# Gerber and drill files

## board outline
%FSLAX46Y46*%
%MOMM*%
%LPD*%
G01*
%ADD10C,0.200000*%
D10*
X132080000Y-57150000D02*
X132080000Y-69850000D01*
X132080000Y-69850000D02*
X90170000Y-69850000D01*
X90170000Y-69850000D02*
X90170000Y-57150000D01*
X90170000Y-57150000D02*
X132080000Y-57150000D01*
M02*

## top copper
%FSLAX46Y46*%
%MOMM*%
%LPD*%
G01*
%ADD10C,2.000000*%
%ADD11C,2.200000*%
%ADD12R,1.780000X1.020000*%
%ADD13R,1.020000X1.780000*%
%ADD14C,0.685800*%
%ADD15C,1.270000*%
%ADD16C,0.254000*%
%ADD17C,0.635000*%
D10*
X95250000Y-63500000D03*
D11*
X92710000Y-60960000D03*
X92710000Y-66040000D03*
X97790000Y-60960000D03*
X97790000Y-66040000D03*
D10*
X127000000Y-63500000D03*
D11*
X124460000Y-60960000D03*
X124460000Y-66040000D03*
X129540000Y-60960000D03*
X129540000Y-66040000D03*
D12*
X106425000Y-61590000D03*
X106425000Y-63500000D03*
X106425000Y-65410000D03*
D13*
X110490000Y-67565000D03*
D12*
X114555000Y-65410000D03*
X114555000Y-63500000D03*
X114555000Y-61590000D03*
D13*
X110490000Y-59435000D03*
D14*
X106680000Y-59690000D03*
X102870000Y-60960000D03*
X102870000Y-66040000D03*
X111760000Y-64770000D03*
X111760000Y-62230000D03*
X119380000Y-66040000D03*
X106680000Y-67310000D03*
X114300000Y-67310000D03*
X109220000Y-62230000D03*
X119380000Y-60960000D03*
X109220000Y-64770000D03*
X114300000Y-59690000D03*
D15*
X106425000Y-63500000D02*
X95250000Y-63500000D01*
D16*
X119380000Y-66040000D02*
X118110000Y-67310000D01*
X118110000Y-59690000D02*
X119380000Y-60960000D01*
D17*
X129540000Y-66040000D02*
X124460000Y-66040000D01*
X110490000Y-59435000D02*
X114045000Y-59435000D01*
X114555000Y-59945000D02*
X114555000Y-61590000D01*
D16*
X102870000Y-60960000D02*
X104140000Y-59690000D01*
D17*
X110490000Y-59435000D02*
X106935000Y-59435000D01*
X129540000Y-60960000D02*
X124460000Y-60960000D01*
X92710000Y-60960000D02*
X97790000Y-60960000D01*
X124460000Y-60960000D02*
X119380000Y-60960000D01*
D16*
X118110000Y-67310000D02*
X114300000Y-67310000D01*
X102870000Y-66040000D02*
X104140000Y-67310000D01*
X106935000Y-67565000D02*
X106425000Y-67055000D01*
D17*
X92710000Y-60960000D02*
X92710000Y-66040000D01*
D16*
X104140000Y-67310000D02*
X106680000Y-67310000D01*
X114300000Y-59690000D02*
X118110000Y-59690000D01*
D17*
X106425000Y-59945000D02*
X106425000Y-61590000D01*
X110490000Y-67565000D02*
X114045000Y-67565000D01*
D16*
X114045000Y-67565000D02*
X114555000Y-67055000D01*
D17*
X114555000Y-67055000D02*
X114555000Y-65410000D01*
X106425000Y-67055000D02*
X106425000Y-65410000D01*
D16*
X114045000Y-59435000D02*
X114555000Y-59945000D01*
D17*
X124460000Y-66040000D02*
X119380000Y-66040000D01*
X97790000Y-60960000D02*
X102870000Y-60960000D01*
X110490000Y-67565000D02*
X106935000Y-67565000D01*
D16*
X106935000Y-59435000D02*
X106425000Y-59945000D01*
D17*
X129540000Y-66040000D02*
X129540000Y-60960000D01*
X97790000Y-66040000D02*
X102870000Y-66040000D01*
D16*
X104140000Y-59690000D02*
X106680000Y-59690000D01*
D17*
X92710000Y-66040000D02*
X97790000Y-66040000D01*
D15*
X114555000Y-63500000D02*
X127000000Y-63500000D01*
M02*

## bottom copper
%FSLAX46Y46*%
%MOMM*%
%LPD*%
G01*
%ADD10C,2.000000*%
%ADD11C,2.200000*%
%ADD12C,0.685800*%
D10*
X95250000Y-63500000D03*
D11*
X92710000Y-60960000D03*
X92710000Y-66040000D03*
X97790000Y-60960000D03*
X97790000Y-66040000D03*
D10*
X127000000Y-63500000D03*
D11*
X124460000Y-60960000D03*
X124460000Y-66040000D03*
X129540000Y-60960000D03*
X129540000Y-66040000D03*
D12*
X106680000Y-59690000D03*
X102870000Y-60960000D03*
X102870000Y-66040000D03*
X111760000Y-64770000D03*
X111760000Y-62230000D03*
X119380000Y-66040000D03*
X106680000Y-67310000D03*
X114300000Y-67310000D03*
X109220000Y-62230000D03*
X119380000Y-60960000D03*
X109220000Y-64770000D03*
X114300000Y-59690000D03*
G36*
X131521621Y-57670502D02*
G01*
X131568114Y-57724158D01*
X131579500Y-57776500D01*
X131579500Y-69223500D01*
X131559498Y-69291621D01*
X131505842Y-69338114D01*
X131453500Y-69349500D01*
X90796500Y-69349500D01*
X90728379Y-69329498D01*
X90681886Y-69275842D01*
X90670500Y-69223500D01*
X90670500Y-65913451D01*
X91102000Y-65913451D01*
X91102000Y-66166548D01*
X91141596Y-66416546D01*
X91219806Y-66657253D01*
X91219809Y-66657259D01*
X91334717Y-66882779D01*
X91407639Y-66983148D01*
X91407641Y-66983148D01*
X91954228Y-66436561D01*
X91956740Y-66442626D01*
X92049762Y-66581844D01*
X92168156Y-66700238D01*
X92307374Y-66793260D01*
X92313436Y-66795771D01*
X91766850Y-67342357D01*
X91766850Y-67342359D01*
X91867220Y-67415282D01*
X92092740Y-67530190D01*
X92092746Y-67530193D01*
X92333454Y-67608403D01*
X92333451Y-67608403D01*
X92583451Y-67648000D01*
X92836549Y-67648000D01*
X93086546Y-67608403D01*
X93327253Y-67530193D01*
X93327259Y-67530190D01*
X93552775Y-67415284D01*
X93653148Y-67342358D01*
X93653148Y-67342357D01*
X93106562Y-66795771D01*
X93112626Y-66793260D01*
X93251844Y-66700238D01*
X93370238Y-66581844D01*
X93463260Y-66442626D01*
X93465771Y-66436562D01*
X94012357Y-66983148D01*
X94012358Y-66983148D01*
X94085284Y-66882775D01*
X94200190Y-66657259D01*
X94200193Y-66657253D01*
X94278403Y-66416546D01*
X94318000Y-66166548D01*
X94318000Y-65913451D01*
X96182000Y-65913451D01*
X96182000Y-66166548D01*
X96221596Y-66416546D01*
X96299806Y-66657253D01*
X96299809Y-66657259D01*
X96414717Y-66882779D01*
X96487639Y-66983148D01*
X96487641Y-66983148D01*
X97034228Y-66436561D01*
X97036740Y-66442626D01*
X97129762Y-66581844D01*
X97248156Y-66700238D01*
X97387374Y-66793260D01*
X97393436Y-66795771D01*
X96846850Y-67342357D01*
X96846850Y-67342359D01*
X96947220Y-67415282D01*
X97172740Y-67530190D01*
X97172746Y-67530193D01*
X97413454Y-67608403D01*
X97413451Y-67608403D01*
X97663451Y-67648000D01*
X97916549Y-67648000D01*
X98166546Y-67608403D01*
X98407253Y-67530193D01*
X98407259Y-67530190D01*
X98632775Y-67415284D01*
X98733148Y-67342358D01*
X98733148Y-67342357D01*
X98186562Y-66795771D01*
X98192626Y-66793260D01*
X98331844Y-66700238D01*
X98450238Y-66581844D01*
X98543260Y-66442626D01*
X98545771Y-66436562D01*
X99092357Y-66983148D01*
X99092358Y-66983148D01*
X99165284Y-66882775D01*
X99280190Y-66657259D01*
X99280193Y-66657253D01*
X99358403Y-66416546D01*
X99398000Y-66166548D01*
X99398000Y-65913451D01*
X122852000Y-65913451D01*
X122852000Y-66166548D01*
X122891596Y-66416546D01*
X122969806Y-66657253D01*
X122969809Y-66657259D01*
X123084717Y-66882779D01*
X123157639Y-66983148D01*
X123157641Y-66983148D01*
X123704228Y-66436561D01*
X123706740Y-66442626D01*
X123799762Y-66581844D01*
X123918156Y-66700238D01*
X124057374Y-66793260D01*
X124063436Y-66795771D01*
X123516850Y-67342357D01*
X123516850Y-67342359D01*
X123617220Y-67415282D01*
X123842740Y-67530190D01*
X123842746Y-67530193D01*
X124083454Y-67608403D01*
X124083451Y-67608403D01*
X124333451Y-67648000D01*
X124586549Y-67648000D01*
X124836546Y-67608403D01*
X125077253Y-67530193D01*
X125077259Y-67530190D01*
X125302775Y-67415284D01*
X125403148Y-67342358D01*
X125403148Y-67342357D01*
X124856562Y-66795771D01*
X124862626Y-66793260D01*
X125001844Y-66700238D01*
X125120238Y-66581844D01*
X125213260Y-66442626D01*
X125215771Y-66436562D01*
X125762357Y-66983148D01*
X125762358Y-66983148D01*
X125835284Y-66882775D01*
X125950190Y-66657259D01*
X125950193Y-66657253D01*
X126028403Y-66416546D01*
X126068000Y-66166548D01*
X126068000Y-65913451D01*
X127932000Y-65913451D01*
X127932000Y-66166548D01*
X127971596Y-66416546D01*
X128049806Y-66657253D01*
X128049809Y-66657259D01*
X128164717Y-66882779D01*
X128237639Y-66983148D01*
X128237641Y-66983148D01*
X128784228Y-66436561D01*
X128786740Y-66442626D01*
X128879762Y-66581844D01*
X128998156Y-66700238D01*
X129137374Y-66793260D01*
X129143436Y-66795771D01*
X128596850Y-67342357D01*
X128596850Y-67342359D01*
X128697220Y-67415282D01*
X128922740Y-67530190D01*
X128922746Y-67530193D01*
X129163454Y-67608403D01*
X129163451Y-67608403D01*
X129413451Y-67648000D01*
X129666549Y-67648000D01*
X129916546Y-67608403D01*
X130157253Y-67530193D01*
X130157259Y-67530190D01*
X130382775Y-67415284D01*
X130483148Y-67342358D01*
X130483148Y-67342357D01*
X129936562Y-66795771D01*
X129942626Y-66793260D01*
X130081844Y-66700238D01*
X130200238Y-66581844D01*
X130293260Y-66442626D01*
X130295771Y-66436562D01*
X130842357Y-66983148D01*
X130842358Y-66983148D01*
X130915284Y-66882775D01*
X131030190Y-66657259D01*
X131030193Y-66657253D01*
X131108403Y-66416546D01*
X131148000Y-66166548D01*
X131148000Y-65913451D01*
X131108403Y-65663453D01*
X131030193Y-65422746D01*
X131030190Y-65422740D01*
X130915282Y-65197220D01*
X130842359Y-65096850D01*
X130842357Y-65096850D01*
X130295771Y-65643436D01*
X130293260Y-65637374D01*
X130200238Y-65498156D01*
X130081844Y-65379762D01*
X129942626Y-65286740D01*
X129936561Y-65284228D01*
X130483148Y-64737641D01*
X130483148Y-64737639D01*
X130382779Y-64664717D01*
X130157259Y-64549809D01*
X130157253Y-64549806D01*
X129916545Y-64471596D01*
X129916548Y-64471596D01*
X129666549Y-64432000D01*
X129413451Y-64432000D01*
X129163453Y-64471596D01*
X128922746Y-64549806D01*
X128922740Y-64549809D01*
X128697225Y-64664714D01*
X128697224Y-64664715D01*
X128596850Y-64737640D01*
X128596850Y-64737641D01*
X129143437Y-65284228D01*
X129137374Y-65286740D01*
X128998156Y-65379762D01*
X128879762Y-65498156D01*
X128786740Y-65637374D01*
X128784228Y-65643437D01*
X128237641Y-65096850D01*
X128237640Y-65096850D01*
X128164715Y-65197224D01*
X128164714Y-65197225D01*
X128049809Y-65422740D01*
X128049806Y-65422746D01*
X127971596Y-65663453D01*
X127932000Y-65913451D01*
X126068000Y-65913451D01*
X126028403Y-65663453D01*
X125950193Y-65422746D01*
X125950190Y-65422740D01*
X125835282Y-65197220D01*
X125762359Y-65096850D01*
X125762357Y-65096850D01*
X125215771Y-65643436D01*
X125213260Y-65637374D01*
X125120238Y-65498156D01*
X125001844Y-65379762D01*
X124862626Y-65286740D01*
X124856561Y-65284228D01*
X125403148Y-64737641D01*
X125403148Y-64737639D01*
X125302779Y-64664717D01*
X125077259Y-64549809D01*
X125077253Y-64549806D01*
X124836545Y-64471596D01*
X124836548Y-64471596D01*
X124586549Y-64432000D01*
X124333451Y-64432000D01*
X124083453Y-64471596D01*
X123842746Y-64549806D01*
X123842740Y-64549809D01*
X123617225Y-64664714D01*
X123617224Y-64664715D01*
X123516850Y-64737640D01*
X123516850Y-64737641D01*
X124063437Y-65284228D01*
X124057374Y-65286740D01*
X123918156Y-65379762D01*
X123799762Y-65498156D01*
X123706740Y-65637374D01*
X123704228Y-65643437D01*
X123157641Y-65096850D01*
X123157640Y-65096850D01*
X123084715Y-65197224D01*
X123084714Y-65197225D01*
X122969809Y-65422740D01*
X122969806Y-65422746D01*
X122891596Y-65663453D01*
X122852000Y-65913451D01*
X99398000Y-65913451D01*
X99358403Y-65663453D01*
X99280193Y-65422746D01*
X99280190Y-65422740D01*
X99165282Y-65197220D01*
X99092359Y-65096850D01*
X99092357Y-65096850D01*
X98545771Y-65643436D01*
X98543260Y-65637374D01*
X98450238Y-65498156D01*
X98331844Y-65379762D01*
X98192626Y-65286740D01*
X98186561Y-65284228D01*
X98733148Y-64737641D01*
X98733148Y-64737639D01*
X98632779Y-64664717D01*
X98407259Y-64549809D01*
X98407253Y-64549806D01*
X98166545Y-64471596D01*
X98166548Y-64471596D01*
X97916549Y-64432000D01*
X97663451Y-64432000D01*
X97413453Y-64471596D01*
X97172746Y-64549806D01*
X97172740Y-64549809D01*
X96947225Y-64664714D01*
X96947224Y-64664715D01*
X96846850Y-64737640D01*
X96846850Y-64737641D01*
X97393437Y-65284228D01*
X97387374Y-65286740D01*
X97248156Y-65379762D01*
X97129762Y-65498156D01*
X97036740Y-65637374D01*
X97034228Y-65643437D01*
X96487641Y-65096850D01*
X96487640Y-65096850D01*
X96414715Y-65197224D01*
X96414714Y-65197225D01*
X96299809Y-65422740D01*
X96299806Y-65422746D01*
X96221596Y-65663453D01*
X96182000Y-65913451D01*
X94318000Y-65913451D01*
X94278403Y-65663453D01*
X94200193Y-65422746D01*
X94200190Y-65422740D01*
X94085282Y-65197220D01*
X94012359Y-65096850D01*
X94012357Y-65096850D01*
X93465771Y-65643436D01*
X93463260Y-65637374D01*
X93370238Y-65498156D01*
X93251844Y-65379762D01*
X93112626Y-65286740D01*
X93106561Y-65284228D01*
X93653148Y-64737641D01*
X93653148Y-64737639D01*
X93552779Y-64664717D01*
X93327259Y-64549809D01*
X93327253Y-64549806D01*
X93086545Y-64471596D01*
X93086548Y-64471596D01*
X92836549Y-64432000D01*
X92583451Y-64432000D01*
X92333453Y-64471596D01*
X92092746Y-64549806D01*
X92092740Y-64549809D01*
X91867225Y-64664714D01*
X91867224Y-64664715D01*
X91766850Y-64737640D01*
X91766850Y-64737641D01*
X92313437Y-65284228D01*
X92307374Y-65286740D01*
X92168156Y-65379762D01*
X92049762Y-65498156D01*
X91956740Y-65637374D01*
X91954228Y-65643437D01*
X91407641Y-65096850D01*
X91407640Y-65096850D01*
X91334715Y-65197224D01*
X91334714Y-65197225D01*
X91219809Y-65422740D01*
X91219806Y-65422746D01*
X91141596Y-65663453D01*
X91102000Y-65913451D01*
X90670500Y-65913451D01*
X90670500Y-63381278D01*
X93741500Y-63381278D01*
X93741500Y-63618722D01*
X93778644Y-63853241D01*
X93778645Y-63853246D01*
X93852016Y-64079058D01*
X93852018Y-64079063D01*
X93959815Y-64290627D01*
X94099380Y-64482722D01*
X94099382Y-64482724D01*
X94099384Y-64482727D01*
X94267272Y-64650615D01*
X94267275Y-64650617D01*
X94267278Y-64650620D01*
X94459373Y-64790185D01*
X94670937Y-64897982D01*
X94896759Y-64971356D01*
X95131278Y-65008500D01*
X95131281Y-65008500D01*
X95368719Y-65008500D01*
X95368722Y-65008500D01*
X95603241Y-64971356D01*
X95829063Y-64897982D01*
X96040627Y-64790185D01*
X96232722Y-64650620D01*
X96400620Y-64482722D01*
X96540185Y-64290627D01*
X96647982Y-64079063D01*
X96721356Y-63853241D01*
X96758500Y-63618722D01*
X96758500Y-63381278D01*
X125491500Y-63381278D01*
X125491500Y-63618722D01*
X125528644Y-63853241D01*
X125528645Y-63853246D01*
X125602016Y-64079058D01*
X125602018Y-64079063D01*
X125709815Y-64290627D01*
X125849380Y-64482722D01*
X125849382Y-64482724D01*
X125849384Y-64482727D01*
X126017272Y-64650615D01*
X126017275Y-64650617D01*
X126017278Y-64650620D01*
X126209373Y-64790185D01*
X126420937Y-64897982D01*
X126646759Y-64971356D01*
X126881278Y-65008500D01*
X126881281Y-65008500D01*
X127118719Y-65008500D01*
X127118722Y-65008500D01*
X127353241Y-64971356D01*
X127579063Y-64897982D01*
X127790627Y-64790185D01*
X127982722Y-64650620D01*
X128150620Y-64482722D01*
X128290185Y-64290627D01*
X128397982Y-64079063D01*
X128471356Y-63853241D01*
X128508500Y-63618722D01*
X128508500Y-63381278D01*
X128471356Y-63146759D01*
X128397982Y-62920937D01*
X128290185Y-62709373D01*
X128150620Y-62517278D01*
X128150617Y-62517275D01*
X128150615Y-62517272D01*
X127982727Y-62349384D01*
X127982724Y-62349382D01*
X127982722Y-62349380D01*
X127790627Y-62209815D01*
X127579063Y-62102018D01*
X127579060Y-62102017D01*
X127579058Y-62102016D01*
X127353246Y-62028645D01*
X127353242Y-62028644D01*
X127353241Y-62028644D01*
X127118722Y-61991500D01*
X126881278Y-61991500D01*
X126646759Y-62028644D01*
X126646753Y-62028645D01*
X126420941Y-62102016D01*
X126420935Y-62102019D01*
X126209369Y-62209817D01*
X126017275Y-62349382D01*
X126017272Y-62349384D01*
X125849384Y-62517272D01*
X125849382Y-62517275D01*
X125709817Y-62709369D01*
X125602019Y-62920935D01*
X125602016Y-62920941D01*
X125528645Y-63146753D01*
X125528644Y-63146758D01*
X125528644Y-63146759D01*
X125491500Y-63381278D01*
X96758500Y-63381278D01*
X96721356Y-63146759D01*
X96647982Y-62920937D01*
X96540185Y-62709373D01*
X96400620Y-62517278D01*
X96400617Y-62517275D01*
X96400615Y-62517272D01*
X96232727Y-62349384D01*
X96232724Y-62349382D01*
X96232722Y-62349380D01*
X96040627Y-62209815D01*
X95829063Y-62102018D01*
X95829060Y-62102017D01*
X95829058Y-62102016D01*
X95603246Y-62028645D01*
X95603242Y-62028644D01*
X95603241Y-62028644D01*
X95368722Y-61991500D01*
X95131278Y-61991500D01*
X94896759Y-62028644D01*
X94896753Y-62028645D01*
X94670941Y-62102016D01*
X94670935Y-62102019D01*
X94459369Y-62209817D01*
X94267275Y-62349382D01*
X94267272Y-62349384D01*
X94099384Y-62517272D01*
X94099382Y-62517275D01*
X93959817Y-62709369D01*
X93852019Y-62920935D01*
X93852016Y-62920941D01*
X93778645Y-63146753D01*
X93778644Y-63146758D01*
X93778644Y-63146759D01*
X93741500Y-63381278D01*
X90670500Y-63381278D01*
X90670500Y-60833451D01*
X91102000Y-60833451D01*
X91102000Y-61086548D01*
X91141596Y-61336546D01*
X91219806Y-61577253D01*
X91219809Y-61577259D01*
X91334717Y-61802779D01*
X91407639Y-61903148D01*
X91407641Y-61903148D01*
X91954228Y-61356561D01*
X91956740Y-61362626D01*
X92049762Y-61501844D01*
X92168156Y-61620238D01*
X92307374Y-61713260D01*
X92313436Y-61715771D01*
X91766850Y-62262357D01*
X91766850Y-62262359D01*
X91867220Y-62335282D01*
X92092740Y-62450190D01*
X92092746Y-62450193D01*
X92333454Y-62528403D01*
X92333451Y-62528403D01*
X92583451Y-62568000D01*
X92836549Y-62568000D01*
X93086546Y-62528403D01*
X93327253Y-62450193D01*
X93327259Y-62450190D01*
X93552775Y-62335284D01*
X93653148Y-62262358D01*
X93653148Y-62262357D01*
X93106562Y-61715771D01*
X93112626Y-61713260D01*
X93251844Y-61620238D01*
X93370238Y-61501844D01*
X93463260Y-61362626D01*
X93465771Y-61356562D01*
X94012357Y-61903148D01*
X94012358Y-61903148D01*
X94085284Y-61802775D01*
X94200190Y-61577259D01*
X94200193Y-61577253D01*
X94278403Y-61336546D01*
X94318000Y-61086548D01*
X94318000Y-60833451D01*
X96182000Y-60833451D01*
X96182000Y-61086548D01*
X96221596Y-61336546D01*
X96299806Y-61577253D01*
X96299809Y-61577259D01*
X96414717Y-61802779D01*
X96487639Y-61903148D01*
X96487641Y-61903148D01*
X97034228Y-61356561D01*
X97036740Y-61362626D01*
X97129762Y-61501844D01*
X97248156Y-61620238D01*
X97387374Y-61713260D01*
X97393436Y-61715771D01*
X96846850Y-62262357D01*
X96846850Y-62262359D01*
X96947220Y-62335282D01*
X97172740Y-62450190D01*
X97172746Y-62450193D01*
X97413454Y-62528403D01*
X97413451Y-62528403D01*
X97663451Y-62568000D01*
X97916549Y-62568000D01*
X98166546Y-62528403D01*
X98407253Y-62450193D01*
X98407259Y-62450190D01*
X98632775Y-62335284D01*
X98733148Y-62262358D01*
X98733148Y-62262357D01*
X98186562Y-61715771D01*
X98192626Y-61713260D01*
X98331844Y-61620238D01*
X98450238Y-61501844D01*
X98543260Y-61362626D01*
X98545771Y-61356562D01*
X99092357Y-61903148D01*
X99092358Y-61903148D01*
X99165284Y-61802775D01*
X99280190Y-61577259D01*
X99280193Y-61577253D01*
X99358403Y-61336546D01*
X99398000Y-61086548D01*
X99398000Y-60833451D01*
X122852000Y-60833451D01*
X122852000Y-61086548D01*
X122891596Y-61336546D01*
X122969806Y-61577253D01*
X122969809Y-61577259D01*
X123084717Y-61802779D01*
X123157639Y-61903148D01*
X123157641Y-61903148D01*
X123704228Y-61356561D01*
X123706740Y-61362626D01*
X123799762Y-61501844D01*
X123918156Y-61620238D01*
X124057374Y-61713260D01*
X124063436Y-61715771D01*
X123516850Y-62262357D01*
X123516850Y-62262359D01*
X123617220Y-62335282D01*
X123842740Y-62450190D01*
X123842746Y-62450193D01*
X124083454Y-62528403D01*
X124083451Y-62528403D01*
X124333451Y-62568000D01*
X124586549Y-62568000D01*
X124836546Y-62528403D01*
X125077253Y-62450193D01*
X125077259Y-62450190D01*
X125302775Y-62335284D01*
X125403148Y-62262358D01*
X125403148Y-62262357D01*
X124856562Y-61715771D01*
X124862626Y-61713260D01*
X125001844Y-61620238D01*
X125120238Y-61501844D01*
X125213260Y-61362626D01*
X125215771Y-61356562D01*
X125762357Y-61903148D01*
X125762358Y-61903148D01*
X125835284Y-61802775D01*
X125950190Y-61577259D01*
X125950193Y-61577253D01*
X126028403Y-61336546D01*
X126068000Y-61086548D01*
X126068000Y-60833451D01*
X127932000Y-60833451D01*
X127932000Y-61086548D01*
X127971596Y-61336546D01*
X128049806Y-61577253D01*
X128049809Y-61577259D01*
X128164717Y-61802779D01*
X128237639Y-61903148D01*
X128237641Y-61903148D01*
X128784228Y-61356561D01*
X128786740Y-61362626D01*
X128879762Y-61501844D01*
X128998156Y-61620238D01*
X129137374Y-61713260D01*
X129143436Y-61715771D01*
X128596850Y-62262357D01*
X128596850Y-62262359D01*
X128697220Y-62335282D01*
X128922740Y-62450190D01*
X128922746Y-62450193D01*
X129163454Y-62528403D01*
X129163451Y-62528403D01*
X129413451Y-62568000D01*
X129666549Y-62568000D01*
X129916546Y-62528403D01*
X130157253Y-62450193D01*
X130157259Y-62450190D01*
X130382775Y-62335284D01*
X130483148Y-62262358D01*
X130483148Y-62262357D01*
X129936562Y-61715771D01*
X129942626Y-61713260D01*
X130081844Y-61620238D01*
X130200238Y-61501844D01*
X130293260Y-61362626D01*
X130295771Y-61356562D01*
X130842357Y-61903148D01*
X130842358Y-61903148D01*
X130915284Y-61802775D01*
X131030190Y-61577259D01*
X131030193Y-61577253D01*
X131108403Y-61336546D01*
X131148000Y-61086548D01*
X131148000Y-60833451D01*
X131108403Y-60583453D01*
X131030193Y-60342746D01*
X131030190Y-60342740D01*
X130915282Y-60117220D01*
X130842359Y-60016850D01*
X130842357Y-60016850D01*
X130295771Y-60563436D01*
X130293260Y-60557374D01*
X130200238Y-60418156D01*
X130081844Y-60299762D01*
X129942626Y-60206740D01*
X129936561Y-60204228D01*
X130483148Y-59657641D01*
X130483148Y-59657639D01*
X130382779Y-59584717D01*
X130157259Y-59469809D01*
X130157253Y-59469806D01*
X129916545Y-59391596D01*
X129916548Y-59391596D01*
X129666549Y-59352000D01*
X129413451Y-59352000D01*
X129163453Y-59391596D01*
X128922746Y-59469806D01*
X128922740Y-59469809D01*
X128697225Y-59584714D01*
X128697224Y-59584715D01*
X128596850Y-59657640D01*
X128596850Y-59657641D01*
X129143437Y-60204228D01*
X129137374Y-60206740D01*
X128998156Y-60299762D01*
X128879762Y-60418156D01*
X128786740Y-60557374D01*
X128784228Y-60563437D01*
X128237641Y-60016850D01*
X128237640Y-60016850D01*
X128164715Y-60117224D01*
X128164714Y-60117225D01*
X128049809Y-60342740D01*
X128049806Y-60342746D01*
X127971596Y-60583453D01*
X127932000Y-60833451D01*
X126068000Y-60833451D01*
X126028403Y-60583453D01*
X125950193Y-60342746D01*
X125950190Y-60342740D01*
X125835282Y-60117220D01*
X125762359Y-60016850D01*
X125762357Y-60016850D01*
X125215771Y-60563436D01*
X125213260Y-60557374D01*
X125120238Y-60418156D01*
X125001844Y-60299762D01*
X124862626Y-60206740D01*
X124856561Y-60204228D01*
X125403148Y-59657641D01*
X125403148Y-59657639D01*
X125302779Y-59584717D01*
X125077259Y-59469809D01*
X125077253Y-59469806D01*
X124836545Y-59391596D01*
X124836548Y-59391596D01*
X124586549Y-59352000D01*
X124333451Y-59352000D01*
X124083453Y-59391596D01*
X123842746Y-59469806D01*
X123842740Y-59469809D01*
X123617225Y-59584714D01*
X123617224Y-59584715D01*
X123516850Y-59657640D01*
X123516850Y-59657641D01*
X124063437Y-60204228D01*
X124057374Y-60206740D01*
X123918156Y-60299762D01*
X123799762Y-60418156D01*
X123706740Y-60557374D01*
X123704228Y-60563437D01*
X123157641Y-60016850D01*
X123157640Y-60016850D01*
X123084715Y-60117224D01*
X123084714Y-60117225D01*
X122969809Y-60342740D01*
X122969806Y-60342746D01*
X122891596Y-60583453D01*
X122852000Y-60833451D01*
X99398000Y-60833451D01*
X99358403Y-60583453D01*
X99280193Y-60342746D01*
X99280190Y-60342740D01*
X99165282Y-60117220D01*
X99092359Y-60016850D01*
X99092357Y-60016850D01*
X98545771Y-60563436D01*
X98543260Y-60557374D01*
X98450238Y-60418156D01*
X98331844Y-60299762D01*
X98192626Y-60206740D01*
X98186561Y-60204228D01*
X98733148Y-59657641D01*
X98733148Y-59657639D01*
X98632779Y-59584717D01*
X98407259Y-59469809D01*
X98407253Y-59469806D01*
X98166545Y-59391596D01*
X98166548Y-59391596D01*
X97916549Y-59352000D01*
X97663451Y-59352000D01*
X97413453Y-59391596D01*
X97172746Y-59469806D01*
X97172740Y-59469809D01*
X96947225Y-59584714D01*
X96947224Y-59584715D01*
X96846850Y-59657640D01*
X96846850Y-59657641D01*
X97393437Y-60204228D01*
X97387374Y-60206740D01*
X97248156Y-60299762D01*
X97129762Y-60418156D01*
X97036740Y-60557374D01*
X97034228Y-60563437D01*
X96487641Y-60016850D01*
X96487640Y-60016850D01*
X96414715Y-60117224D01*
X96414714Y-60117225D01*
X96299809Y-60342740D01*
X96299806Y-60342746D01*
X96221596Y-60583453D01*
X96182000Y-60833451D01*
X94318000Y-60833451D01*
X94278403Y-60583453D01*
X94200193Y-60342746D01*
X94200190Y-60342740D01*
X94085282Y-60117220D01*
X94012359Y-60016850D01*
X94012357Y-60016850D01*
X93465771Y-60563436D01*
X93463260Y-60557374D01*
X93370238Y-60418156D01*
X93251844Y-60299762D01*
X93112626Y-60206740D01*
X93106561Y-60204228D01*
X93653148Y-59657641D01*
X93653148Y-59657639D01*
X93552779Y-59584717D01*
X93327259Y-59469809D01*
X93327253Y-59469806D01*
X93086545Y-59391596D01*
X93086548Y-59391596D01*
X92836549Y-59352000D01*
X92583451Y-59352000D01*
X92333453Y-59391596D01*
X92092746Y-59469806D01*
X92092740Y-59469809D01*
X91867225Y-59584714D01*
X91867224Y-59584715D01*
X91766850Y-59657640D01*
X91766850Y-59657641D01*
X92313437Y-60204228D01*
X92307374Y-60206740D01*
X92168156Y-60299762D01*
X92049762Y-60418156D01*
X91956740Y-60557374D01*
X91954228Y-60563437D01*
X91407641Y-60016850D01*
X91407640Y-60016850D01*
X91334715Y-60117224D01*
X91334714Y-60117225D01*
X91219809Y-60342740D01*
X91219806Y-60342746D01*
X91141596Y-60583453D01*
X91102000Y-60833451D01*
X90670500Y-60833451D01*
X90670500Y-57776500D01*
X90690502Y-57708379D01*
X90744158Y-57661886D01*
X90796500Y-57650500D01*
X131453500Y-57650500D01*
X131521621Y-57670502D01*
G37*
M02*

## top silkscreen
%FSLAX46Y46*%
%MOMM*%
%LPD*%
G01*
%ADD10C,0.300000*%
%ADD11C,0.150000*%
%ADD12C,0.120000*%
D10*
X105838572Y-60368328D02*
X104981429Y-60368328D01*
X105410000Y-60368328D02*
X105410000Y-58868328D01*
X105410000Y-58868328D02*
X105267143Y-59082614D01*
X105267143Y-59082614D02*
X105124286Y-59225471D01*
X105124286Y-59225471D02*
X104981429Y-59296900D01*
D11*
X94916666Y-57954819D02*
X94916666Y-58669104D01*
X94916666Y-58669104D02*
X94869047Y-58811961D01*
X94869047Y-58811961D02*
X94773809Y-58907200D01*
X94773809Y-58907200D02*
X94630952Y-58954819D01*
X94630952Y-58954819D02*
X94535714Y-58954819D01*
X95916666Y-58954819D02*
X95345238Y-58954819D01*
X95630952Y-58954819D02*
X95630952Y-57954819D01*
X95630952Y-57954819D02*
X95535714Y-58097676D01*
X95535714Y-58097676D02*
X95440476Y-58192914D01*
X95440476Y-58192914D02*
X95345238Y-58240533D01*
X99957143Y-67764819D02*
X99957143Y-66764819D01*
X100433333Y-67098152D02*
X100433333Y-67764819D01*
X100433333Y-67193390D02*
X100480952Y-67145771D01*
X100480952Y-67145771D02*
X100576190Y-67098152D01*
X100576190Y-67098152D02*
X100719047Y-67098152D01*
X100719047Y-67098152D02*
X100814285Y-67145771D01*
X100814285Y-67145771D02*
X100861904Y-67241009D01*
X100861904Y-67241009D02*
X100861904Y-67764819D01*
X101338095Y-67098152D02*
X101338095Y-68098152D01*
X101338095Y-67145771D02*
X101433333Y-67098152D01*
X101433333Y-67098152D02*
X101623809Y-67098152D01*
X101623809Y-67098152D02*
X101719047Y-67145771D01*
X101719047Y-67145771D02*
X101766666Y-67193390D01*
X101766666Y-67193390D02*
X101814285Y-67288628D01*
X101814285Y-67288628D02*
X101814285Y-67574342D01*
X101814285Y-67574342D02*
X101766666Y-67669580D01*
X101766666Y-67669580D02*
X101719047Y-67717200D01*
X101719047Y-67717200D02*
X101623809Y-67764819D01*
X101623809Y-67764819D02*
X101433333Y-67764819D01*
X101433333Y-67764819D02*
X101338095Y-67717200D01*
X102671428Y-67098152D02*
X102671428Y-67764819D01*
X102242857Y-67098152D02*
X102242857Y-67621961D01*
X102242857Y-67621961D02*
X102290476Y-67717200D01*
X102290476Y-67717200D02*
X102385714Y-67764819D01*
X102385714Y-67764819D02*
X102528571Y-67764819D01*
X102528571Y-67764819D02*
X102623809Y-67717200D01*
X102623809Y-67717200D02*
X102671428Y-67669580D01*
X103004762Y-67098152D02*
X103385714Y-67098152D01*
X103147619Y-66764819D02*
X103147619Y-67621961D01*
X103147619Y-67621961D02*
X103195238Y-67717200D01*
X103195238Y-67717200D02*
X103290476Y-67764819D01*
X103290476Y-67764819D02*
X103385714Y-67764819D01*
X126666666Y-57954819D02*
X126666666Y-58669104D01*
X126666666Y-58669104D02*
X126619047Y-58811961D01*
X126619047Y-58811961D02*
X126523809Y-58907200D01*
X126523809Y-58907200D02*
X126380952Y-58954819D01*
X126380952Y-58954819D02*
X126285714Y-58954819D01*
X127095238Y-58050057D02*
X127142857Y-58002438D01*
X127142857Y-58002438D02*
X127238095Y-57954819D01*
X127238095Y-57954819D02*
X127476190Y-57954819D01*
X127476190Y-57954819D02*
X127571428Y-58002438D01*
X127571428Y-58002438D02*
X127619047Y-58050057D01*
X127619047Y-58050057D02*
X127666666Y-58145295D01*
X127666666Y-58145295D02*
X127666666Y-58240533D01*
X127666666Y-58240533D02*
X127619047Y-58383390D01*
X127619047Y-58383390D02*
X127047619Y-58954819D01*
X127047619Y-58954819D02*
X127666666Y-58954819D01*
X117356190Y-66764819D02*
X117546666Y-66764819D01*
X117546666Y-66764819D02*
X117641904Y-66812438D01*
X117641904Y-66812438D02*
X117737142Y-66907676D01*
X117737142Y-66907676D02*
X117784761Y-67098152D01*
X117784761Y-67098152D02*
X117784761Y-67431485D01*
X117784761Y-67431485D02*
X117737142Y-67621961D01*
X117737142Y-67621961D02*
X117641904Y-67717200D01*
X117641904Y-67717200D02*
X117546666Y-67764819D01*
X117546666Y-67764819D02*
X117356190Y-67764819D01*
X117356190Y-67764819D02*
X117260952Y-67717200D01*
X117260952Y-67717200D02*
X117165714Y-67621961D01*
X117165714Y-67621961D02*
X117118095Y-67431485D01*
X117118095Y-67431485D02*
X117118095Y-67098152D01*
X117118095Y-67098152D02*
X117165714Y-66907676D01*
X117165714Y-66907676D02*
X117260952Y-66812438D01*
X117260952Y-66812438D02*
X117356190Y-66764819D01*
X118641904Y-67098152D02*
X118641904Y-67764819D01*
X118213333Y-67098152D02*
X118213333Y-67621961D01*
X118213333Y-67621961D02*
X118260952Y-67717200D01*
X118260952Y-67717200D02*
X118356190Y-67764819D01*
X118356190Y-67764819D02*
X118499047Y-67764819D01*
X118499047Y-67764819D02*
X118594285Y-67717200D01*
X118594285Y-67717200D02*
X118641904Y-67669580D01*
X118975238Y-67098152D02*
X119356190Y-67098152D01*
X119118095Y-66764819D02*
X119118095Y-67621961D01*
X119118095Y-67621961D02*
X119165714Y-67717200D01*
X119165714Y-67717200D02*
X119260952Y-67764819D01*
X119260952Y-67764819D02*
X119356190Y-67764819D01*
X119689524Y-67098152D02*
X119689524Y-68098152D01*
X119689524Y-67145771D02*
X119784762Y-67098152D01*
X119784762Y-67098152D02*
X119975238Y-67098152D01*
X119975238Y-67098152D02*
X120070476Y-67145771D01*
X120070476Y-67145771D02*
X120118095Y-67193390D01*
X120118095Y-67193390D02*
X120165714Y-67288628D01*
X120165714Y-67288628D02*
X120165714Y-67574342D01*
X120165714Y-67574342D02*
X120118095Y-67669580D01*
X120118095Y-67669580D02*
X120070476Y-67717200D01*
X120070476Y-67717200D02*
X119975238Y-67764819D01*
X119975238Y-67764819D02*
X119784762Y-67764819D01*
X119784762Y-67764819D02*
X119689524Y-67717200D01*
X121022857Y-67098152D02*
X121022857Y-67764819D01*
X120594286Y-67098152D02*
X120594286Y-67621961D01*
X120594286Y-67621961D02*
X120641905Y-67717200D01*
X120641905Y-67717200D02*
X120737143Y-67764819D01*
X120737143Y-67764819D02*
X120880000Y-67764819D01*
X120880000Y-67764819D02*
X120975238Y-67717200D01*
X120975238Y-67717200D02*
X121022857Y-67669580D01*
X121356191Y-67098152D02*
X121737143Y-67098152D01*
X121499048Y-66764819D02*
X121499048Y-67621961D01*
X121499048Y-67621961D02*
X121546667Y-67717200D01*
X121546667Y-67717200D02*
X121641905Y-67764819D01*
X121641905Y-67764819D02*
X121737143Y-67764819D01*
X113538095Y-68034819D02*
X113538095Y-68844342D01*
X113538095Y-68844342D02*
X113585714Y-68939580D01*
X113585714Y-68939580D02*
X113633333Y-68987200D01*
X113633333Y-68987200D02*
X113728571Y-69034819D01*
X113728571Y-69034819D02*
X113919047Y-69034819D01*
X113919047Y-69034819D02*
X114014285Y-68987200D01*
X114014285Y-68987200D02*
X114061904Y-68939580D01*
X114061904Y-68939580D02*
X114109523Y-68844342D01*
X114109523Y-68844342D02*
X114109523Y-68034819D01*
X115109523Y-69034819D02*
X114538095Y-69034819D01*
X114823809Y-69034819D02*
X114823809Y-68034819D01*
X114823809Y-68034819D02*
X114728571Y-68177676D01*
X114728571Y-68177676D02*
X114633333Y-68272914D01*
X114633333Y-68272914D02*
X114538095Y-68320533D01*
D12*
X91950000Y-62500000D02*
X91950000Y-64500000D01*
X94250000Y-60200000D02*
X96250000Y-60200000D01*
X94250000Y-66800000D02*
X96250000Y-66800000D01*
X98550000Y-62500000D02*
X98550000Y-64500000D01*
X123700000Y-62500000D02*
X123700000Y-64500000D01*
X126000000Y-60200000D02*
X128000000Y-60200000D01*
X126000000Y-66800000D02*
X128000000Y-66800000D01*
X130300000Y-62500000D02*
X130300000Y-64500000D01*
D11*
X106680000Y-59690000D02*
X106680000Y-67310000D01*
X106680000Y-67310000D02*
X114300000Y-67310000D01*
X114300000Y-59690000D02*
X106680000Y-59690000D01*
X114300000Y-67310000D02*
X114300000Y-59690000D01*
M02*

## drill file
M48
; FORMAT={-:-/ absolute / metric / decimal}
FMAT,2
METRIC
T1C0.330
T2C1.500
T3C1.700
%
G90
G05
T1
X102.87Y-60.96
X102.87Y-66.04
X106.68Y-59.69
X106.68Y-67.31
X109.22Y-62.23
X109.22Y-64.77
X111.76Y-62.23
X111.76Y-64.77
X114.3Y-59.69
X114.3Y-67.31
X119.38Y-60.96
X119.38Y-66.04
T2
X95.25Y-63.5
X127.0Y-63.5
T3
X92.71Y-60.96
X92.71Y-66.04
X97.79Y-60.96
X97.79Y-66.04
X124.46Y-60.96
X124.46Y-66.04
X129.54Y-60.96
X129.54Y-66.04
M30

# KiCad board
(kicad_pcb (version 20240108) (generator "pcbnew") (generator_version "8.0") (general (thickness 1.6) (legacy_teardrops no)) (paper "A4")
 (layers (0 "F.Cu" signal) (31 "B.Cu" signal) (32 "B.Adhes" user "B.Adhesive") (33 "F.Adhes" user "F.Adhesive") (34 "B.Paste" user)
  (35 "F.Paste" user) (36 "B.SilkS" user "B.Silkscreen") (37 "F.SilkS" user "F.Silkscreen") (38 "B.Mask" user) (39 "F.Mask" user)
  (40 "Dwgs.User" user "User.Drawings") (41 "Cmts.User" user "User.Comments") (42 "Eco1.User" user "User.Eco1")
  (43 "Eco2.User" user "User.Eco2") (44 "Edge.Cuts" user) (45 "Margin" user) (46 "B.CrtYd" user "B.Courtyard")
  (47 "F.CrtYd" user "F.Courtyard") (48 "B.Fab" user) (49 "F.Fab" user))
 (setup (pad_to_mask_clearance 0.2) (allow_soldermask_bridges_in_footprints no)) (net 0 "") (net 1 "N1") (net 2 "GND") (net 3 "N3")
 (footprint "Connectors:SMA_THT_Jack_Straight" (layer "F.Cu") (at 95.25 63.5)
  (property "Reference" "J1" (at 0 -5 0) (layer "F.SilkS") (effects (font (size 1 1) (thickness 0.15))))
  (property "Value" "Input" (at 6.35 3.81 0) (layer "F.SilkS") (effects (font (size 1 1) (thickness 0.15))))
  (fp_line (start -3.3 -1) (end -3.3 1) (stroke (width 0.12) (type solid)) (layer "F.SilkS"))
  (fp_line (start -1 -3.3) (end 1 -3.3) (stroke (width 0.12) (type solid)) (layer "F.SilkS"))
  (fp_line (start -1 3.3) (end 1 3.3) (stroke (width 0.12) (type solid)) (layer "F.SilkS"))
  (fp_line (start 3.3 -1) (end 3.3 1) (stroke (width 0.12) (type solid)) (layer "F.SilkS"))
  (pad "1" thru_hole circle (at 0 0) (size 2 2) (drill 1.5) (layers "*.Cu" "*.Mask") (remove_unused_layers no) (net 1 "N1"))
  (pad "2" thru_hole circle (at -2.54 -2.54) (size 2.2 2.2) (drill 1.7) (layers "*.Cu" "*.Mask") (remove_unused_layers no) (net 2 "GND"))
  (pad "2" thru_hole circle (at -2.54 2.54) (size 2.2 2.2) (drill 1.7) (layers "*.Cu" "*.Mask") (remove_unused_layers no) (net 2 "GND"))
  (pad "2" thru_hole circle (at 2.54 -2.54) (size 2.2 2.2) (drill 1.7) (layers "*.Cu" "*.Mask") (remove_unused_layers no) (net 2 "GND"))
  (pad "2" thru_hole circle (at 2.54 2.54) (size 2.2 2.2) (drill 1.7) (layers "*.Cu" "*.Mask") (remove_unused_layers no) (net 2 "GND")))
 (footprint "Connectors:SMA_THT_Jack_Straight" (layer "F.Cu") (at 127 63.5)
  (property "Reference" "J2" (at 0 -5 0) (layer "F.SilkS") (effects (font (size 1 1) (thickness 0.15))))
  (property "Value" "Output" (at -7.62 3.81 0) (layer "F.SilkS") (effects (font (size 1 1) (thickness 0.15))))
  (fp_line (start -3.3 -1) (end -3.3 1) (stroke (width 0.12) (type solid)) (layer "F.SilkS"))
  (fp_line (start -1 -3.3) (end 1 -3.3) (stroke (width 0.12) (type solid)) (layer "F.SilkS"))
  (fp_line (start -1 3.3) (end 1 3.3) (stroke (width 0.12) (type solid)) (layer "F.SilkS"))
  (fp_line (start 3.3 -1) (end 3.3 1) (stroke (width 0.12) (type solid)) (layer "F.SilkS"))
  (pad "1" thru_hole circle (at 0 0) (size 2 2) (drill 1.5) (layers "*.Cu" "*.Mask") (remove_unused_layers no) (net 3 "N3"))
  (pad "2" thru_hole circle (at -2.54 -2.54) (size 2.2 2.2) (drill 1.7) (layers "*.Cu" "*.Mask") (remove_unused_layers no) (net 2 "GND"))
  (pad "2" thru_hole circle (at -2.54 2.54) (size 2.2 2.2) (drill 1.7) (layers "*.Cu" "*.Mask") (remove_unused_layers no) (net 2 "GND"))
  (pad "2" thru_hole circle (at 2.54 -2.54) (size 2.2 2.2) (drill 1.7) (layers "*.Cu" "*.Mask") (remove_unused_layers no) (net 2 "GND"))
  (pad "2" thru_hole circle (at 2.54 2.54) (size 2.2 2.2) (drill 1.7) (layers "*.Cu" "*.Mask") (remove_unused_layers no) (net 2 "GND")))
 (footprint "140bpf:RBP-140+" (layer "F.Cu") (at 110.49 63.5 -90)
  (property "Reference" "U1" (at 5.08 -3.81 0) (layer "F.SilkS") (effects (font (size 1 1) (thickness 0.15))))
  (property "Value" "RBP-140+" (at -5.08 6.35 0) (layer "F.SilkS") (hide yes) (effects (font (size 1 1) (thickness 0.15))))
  (fp_line (start -3.81 3.81) (end 3.81 3.81) (stroke (width 0.15) (type solid)) (layer "F.SilkS"))
  (fp_line (start 3.81 3.81) (end 3.81 -3.81) (stroke (width 0.15) (type solid)) (layer "F.SilkS"))
  (fp_line (start -3.81 -3.81) (end -3.81 3.81) (stroke (width 0.15) (type solid)) (layer "F.SilkS"))
  (fp_line (start 3.81 -3.81) (end -3.81 -3.81) (stroke (width 0.15) (type solid)) (layer "F.SilkS"))
  (pad "1" smd rect (at -1.91 4.065 270) (size 1.02 1.78) (layers "F.Cu" "F.Paste" "F.Mask") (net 2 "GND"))
  (pad "2" smd rect (at 0 4.065 270) (size 1.02 1.78) (layers "F.Cu" "F.Paste" "F.Mask") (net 1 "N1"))
  (pad "3" smd rect (at 1.91 4.065 90) (size 1.02 1.78) (layers "F.Cu" "F.Paste" "F.Mask") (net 2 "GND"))
  (pad "4" smd rect (at 4.065 0) (size 1.02 1.78) (layers "F.Cu" "F.Paste" "F.Mask") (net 2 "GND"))
  (pad "5" smd rect (at 1.91 -4.065 270) (size 1.02 1.78) (layers "F.Cu" "F.Paste" "F.Mask") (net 2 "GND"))
  (pad "6" smd rect (at 0 -4.065 270) (size 1.02 1.78) (layers "F.Cu" "F.Paste" "F.Mask") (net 3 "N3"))
  (pad "7" smd rect (at -1.91 -4.065 270) (size 1.02 1.78) (layers "F.Cu" "F.Paste" "F.Mask") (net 2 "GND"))
  (pad "8" smd rect (at -4.065 0) (size 1.02 1.78) (layers "F.Cu" "F.Paste" "F.Mask") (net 2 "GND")))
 (gr_line (start 132.08 57.15) (end 132.08 69.85) (stroke (width 0.2) (type solid)) (layer "Edge.Cuts"))
 (gr_line (start 132.08 69.85) (end 90.17 69.85) (stroke (width 0.2) (type solid)) (layer "Edge.Cuts"))
 (gr_line (start 90.17 69.85) (end 90.17 57.15) (stroke (width 0.2) (type solid)) (layer "Edge.Cuts"))
 (gr_line (start 90.17 57.15) (end 132.08 57.15) (stroke (width 0.2) (type solid)) (layer "Edge.Cuts"))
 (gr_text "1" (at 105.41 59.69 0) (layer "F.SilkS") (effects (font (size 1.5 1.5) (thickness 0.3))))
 (segment (start 106.425 63.5) (end 95.25 63.5) (width 1.27) (layer "F.Cu") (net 1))
 (segment (start 119.38 66.04) (end 118.11 67.31) (width 0.254) (layer "F.Cu") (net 2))
 (segment (start 118.11 59.69) (end 119.38 60.96) (width 0.254) (layer "F.Cu") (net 2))
 (segment (start 129.54 66.04) (end 124.46 66.04) (width 0.635) (layer "F.Cu") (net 2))
 (segment (start 110.49 59.435) (end 114.045 59.435) (width 0.635) (layer "F.Cu") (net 2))
 (segment (start 114.555 59.945) (end 114.555 61.59) (width 0.635) (layer "F.Cu") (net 2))
 (segment (start 102.87 60.96) (end 104.14 59.69) (width 0.254) (layer "F.Cu") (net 2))
 (segment (start 110.49 59.435) (end 106.935 59.435) (width 0.635) (layer "F.Cu") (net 2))
 (segment (start 129.54 60.96) (end 124.46 60.96) (width 0.635) (layer "F.Cu") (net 2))
 (segment (start 92.71 60.96) (end 97.79 60.96) (width 0.635) (layer "F.Cu") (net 2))
 (segment (start 124.46 60.96) (end 119.38 60.96) (width 0.635) (layer "F.Cu") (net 2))
 (segment (start 118.11 67.31) (end 114.3 67.31) (width 0.254) (layer "F.Cu") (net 2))
 (segment (start 102.87 66.04) (end 104.14 67.31) (width 0.254) (layer "F.Cu") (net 2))
 (segment (start 106.935 67.565) (end 106.425 67.055) (width 0.254) (layer "F.Cu") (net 2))
 (segment (start 92.71 60.96) (end 92.71 66.04) (width 0.635) (layer "F.Cu") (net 2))
 (segment (start 104.14 67.31) (end 106.68 67.31) (width 0.254) (layer "F.Cu") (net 2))
 (segment (start 114.3 59.69) (end 118.11 59.69) (width 0.254) (layer "F.Cu") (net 2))
 (segment (start 106.425 59.945) (end 106.425 61.59) (width 0.635) (layer "F.Cu") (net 2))
 (segment (start 110.49 67.565) (end 114.045 67.565) (width 0.635) (layer "F.Cu") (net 2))
 (segment (start 114.045 67.565) (end 114.555 67.055) (width 0.254) (layer "F.Cu") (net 2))
 (segment (start 114.555 67.055) (end 114.555 65.41) (width 0.635) (layer "F.Cu") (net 2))
 (segment (start 106.425 67.055) (end 106.425 65.41) (width 0.635) (layer "F.Cu") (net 2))
 (segment (start 114.045 59.435) (end 114.555 59.945) (width 0.254) (layer "F.Cu") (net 2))
 (segment (start 124.46 66.04) (end 119.38 66.04) (width 0.635) (layer "F.Cu") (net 2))
 (segment (start 97.79 60.96) (end 102.87 60.96) (width 0.635) (layer "F.Cu") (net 2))
 (segment (start 110.49 67.565) (end 106.935 67.565) (width 0.635) (layer "F.Cu") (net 2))
 (segment (start 106.935 59.435) (end 106.425 59.945) (width 0.254) (layer "F.Cu") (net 2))
 (segment (start 129.54 66.04) (end 129.54 60.96) (width 0.635) (layer "F.Cu") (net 2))
 (segment (start 97.79 66.04) (end 102.87 66.04) (width 0.635) (layer "F.Cu") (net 2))
 (segment (start 104.14 59.69) (end 106.68 59.69) (width 0.254) (layer "F.Cu") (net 2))
 (segment (start 92.71 66.04) (end 97.79 66.04) (width 0.635) (layer "F.Cu") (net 2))
 (via (at 106.68 59.69) (size 0.6858) (drill 0.3302) (layers "F.Cu" "B.Cu") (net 2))
 (via (at 102.87 60.96) (size 0.6858) (drill 0.3302) (layers "F.Cu" "B.Cu") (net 2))
 (via (at 102.87 66.04) (size 0.6858) (drill 0.3302) (layers "F.Cu" "B.Cu") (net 2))
 (via (at 111.76 64.77) (size 0.6858) (drill 0.3302) (layers "F.Cu" "B.Cu") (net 2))
 (via (at 111.76 62.23) (size 0.6858) (drill 0.3302) (layers "F.Cu" "B.Cu") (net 2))
 (via (at 119.38 66.04) (size 0.6858) (drill 0.3302) (layers "F.Cu" "B.Cu") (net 2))
 (via (at 106.68 67.31) (size 0.6858) (drill 0.3302) (layers "F.Cu" "B.Cu") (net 2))
 (via (at 114.3 67.31) (size 0.6858) (drill 0.3302) (layers "F.Cu" "B.Cu") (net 2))
 (via (at 109.22 62.23) (size 0.6858) (drill 0.3302) (layers "F.Cu" "B.Cu") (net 2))
 (via (at 119.38 60.96) (size 0.6858) (drill 0.3302) (layers "F.Cu" "B.Cu") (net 2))
 (via (at 109.22 64.77) (size 0.6858) (drill 0.3302) (layers "F.Cu" "B.Cu") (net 2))
 (via (at 114.3 59.69) (size 0.6858) (drill 0.3302) (layers "F.Cu" "B.Cu") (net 2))
 (segment (start 114.555 63.5) (end 127 63.5) (width 1.27) (layer "F.Cu") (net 3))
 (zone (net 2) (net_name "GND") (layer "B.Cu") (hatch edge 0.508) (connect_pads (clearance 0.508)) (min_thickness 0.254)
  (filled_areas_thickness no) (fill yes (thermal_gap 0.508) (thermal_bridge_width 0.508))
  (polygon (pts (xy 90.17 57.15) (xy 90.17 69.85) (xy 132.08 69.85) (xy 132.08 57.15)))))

